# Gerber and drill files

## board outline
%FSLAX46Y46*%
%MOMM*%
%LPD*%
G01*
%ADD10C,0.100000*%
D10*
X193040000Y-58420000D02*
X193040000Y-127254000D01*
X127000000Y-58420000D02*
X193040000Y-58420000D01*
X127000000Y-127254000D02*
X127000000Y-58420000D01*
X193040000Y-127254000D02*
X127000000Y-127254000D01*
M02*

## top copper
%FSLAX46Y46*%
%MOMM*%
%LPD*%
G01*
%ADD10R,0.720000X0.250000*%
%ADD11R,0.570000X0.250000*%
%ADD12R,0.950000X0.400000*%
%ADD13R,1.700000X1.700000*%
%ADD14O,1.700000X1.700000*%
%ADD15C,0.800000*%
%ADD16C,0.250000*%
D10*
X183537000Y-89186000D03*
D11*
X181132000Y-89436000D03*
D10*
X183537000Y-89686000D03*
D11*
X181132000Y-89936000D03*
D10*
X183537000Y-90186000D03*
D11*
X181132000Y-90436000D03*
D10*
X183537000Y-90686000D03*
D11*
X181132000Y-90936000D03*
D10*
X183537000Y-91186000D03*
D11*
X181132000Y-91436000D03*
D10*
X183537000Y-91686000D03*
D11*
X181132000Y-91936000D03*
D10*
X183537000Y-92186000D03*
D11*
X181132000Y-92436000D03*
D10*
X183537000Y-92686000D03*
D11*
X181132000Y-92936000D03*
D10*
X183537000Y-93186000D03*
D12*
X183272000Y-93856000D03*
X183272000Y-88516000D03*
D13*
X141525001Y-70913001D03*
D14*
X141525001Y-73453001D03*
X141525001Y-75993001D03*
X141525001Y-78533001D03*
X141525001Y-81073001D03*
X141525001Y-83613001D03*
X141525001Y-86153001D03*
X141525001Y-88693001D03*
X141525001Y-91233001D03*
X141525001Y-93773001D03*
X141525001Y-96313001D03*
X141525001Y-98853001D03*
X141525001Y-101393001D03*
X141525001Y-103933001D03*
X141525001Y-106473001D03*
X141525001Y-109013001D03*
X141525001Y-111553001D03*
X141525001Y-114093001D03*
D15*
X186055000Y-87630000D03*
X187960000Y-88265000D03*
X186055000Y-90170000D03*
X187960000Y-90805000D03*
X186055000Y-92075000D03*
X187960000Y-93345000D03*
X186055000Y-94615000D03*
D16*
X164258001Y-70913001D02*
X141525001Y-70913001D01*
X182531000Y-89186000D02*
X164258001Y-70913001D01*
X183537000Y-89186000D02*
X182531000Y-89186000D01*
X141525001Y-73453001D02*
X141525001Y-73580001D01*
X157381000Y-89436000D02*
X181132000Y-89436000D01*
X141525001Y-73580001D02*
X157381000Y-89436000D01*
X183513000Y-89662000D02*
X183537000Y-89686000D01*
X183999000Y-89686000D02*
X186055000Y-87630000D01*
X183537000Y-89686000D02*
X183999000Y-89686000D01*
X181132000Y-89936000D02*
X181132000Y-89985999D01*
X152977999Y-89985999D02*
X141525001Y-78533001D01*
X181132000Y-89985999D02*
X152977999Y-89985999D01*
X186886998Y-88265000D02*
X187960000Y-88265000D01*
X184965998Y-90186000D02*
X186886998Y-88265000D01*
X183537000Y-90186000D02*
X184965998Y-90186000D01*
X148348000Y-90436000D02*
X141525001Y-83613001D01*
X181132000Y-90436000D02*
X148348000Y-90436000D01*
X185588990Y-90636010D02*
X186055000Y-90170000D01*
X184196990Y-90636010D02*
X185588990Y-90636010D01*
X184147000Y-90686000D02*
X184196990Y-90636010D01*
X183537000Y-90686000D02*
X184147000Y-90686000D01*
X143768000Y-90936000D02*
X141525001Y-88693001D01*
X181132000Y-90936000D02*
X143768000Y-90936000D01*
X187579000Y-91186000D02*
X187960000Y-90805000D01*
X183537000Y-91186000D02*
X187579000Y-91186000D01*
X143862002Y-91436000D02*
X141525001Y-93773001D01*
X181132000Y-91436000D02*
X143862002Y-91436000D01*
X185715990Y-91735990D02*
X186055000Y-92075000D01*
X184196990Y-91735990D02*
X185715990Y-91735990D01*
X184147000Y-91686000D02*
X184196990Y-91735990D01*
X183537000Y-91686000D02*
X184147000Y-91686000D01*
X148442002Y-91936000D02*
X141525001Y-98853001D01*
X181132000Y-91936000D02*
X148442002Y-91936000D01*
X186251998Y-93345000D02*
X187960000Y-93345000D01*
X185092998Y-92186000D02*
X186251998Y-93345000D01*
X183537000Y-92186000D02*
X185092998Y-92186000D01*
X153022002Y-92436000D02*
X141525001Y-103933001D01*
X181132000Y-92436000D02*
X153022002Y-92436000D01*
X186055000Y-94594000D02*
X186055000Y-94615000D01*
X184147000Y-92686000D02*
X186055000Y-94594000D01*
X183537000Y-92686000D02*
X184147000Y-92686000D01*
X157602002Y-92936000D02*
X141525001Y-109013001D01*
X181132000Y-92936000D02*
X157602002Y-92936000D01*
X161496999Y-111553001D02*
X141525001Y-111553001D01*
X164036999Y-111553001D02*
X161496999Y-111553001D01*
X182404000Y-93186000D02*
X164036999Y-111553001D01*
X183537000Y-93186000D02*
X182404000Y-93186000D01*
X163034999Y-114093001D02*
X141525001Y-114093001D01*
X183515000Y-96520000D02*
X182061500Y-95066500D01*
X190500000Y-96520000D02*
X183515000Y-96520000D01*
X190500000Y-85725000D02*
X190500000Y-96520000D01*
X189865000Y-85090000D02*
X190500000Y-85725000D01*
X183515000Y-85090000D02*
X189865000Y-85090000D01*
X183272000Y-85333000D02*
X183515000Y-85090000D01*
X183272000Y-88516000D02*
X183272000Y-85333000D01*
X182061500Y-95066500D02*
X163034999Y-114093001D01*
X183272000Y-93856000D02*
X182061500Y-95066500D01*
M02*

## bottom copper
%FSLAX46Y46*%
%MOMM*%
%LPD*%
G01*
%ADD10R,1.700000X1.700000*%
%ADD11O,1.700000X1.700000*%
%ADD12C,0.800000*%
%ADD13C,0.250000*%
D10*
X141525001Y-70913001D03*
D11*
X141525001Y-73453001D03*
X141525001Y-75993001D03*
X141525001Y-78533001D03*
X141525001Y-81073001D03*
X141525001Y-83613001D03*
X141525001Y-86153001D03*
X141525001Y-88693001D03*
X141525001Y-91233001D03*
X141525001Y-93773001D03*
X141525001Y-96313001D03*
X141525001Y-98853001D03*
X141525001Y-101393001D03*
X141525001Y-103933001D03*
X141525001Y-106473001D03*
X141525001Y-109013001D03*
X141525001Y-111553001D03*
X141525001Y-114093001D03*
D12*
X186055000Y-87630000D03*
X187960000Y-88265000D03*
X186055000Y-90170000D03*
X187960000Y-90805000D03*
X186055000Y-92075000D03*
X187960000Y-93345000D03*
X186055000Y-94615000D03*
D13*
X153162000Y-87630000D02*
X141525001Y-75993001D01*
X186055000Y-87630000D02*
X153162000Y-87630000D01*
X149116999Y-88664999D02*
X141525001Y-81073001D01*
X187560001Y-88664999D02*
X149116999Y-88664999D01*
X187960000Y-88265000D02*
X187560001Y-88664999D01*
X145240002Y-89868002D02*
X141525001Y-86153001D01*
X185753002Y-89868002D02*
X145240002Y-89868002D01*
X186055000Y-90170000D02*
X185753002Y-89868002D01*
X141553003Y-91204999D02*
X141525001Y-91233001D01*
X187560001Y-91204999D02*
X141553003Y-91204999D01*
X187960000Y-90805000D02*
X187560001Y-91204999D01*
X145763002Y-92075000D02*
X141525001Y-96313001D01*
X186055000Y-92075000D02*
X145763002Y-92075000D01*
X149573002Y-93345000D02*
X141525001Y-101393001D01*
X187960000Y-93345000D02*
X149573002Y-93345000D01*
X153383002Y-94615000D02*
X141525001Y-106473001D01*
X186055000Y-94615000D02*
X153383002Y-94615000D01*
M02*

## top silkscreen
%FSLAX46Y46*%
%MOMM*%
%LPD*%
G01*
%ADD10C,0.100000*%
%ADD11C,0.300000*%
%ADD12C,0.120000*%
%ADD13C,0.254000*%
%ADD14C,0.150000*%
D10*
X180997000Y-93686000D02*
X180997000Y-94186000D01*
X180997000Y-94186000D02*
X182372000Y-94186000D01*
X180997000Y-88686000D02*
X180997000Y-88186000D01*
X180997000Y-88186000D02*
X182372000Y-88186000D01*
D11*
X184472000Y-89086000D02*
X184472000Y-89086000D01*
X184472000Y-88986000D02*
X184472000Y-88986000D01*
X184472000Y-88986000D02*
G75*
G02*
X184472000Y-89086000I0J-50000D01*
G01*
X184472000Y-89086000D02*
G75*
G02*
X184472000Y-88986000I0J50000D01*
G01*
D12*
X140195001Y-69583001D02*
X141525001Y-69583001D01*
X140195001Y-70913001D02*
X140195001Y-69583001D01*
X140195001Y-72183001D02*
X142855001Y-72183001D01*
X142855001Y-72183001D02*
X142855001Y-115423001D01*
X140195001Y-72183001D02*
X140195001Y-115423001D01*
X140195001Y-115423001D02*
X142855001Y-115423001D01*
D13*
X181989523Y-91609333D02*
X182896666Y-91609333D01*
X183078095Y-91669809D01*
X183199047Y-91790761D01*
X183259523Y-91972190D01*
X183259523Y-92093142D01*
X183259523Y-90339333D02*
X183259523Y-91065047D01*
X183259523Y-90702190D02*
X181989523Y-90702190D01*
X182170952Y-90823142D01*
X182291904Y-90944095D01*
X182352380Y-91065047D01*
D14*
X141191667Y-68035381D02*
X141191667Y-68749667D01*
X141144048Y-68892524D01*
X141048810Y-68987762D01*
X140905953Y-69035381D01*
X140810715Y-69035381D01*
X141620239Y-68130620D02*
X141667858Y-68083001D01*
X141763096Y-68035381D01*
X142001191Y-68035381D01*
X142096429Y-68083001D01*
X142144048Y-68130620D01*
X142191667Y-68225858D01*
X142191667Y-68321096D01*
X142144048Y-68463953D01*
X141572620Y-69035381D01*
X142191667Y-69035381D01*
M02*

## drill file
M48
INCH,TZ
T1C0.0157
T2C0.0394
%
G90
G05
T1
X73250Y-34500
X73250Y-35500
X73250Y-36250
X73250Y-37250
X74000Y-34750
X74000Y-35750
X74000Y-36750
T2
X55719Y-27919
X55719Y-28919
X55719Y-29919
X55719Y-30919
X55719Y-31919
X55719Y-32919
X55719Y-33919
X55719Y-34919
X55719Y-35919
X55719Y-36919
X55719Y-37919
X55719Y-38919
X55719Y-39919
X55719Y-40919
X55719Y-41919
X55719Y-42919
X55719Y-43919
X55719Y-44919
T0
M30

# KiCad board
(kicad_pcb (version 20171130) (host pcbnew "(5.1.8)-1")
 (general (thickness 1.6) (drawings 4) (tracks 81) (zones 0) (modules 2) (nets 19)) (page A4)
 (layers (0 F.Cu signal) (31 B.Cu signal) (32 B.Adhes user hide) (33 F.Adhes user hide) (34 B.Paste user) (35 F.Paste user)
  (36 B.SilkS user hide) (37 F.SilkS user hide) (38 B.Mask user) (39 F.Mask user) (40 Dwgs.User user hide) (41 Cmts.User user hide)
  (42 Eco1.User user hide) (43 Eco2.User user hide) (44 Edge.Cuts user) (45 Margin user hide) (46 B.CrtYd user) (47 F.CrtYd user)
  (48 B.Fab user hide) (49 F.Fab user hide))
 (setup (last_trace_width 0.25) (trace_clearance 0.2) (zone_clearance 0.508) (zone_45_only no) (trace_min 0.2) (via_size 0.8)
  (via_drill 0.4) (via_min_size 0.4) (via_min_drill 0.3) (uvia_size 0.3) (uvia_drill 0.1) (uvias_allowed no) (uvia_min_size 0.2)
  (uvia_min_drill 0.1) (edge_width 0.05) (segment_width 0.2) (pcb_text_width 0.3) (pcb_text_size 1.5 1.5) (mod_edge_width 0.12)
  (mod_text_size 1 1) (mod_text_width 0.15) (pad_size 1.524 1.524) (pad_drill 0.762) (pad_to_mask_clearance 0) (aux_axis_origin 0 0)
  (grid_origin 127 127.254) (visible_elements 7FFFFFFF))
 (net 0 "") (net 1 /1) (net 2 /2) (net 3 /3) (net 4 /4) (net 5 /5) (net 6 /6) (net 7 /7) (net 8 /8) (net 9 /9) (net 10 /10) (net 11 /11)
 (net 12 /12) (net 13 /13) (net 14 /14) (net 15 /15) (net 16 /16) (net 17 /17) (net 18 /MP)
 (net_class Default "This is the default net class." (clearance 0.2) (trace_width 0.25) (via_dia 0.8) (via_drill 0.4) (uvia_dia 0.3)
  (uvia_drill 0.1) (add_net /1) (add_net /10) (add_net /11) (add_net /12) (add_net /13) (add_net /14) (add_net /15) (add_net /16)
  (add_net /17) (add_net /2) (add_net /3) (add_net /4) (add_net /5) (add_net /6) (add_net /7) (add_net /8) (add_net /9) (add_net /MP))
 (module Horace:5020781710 (layer F.Cu) (at 182.372 91.186 90)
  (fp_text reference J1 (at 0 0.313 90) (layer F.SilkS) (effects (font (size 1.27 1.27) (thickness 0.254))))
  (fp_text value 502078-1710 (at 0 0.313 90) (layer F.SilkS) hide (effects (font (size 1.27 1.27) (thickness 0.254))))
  (fp_line (start -2.5 -1.375) (end -3 -1.375) (layer F.SilkS) (width 0.1))
  (fp_line (start -3 -1.375) (end -3 0) (layer F.SilkS) (width 0.1))
  (fp_line (start 2.5 -1.375) (end 3 -1.375) (layer F.SilkS) (width 0.1))
  (fp_line (start 3 -1.375) (end 3 0) (layer F.SilkS) (width 0.1))
  (fp_line (start 2.1 2.1) (end 2.1 2.1) (layer F.SilkS) (width 0.3))
  (fp_line (start 2.2 2.1) (end 2.2 2.1) (layer F.SilkS) (width 0.3))
  (fp_arc (start 2.15 2.1) (end 2.1 2.1) (angle -180) (layer F.SilkS) (width 0.3))
  (fp_arc (start 2.15 2.1) (end 2.2 2.1) (angle -180) (layer F.SilkS) (width 0.3))
  (pad 1 smd rect (at 2 1.165 90) (size 0.25 0.72) (layers F.Cu F.Paste F.Mask) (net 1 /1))
  (pad 2 smd rect (at 1.75 -1.24 90) (size 0.25 0.57) (layers F.Cu F.Paste F.Mask) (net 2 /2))
  (pad 3 smd rect (at 1.5 1.165 90) (size 0.25 0.72) (layers F.Cu F.Paste F.Mask) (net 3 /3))
  (pad 4 smd rect (at 1.25 -1.24 90) (size 0.25 0.57) (layers F.Cu F.Paste F.Mask) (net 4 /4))
  (pad 5 smd rect (at 1 1.165 90) (size 0.25 0.72) (layers F.Cu F.Paste F.Mask) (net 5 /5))
  (pad 6 smd rect (at 0.75 -1.24 90) (size 0.25 0.57) (layers F.Cu F.Paste F.Mask) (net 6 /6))
  (pad 7 smd rect (at 0.5 1.165 90) (size 0.25 0.72) (layers F.Cu F.Paste F.Mask) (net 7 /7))
  (pad 8 smd rect (at 0.25 -1.24 90) (size 0.25 0.57) (layers F.Cu F.Paste F.Mask) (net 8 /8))
  (pad 9 smd rect (at 0 1.165 90) (size 0.25 0.72) (layers F.Cu F.Paste F.Mask) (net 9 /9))
  (pad 10 smd rect (at -0.25 -1.24 90) (size 0.25 0.57) (layers F.Cu F.Paste F.Mask) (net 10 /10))
  (pad 11 smd rect (at -0.5 1.165 90) (size 0.25 0.72) (layers F.Cu F.Paste F.Mask) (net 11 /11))
  (pad 12 smd rect (at -0.75 -1.24 90) (size 0.25 0.57) (layers F.Cu F.Paste F.Mask) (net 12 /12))
  (pad 13 smd rect (at -1 1.165 90) (size 0.25 0.72) (layers F.Cu F.Paste F.Mask) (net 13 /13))
  (pad 14 smd rect (at -1.25 -1.24 90) (size 0.25 0.57) (layers F.Cu F.Paste F.Mask) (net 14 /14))
  (pad 15 smd rect (at -1.5 1.165 90) (size 0.25 0.72) (layers F.Cu F.Paste F.Mask) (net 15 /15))
  (pad 16 smd rect (at -1.75 -1.24 90) (size 0.25 0.57) (layers F.Cu F.Paste F.Mask) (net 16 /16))
  (pad 17 smd rect (at -2 1.165 90) (size 0.25 0.72) (layers F.Cu F.Paste F.Mask) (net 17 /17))
  (pad MP1 smd rect (at -2.67 0.9 90) (size 0.4 0.95) (layers F.Cu F.Paste F.Mask) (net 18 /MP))
  (pad MP2 smd rect (at 2.67 0.9 90) (size 0.4 0.95) (layers F.Cu F.Paste F.Mask) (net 18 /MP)))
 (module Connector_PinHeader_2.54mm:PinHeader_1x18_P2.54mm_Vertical (layer F.Cu) (at 141.525001 70.913001)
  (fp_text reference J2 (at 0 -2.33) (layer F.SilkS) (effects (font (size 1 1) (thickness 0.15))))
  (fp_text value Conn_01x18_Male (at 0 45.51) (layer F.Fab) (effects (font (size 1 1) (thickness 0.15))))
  (fp_line (start -1.33 -1.33) (end 0 -1.33) (layer F.SilkS) (width 0.12))
  (fp_line (start -1.33 0) (end -1.33 -1.33) (layer F.SilkS) (width 0.12))
  (fp_line (start -1.33 1.27) (end 1.33 1.27) (layer F.SilkS) (width 0.12))
  (fp_line (start 1.33 1.27) (end 1.33 44.51) (layer F.SilkS) (width 0.12))
  (fp_line (start -1.33 1.27) (end -1.33 44.51) (layer F.SilkS) (width 0.12))
  (fp_line (start -1.33 44.51) (end 1.33 44.51) (layer F.SilkS) (width 0.12))
  (pad 1 thru_hole rect (at 0 0) (size 1.7 1.7) (drill 1) (layers *.Cu *.Mask) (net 1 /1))
  (pad 2 thru_hole oval (at 0 2.54) (size 1.7 1.7) (drill 1) (layers *.Cu *.Mask) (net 2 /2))
  (pad 3 thru_hole oval (at 0 5.08) (size 1.7 1.7) (drill 1) (layers *.Cu *.Mask) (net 3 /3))
  (pad 4 thru_hole oval (at 0 7.62) (size 1.7 1.7) (drill 1) (layers *.Cu *.Mask) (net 4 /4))
  (pad 5 thru_hole oval (at 0 10.16) (size 1.7 1.7) (drill 1) (layers *.Cu *.Mask) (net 5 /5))
  (pad 6 thru_hole oval (at 0 12.7) (size 1.7 1.7) (drill 1) (layers *.Cu *.Mask) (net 6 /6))
  (pad 7 thru_hole oval (at 0 15.24) (size 1.7 1.7) (drill 1) (layers *.Cu *.Mask) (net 7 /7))
  (pad 8 thru_hole oval (at 0 17.78) (size 1.7 1.7) (drill 1) (layers *.Cu *.Mask) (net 8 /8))
  (pad 9 thru_hole oval (at 0 20.32) (size 1.7 1.7) (drill 1) (layers *.Cu *.Mask) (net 9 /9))
  (pad 10 thru_hole oval (at 0 22.86) (size 1.7 1.7) (drill 1) (layers *.Cu *.Mask) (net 10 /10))
  (pad 11 thru_hole oval (at 0 25.4) (size 1.7 1.7) (drill 1) (layers *.Cu *.Mask) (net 11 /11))
  (pad 12 thru_hole oval (at 0 27.94) (size 1.7 1.7) (drill 1) (layers *.Cu *.Mask) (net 12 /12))
  (pad 13 thru_hole oval (at 0 30.48) (size 1.7 1.7) (drill 1) (layers *.Cu *.Mask) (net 13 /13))
  (pad 14 thru_hole oval (at 0 33.02) (size 1.7 1.7) (drill 1) (layers *.Cu *.Mask) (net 14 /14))
  (pad 15 thru_hole oval (at 0 35.56) (size 1.7 1.7) (drill 1) (layers *.Cu *.Mask) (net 15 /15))
  (pad 16 thru_hole oval (at 0 38.1) (size 1.7 1.7) (drill 1) (layers *.Cu *.Mask) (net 16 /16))
  (pad 17 thru_hole oval (at 0 40.64) (size 1.7 1.7) (drill 1) (layers *.Cu *.Mask) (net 17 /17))
  (pad 18 thru_hole oval (at 0 43.18) (size 1.7 1.7) (drill 1) (layers *.Cu *.Mask) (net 18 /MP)))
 (gr_line (start 193.04 58.42) (end 193.04 127.254) (layer Edge.Cuts) (width 0.1))
 (gr_line (start 127 58.42) (end 193.04 58.42) (layer Edge.Cuts) (width 0.1))
 (gr_line (start 127 127.254) (end 127 58.42) (layer Edge.Cuts) (width 0.1))
 (gr_line (start 193.04 127.254) (end 127 127.254) (layer Edge.Cuts) (width 0.1))
 (segment (start 164.258001 70.913001) (end 141.525001 70.913001) (width 0.25) (layer F.Cu) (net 1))
 (segment (start 182.531 89.186) (end 164.258001 70.913001) (width 0.25) (layer F.Cu) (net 1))
 (segment (start 183.537 89.186) (end 182.531 89.186) (width 0.25) (layer F.Cu) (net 1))
 (segment (start 141.525001 73.453001) (end 141.525001 73.580001) (width 0.25) (layer F.Cu) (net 2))
 (segment (start 157.381 89.436) (end 181.132 89.436) (width 0.25) (layer F.Cu) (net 2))
 (segment (start 141.525001 73.580001) (end 157.381 89.436) (width 0.25) (layer F.Cu) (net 2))
 (via (at 186.055 87.63) (size 0.8) (drill 0.4) (layers F.Cu B.Cu) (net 3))
 (segment (start 183.513 89.662) (end 183.537 89.686) (width 0.25) (layer F.Cu) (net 3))
 (segment (start 183.999 89.686) (end 186.055 87.63) (width 0.25) (layer F.Cu) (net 3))
 (segment (start 183.537 89.686) (end 183.999 89.686) (width 0.25) (layer F.Cu) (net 3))
 (segment (start 153.162 87.63) (end 141.525001 75.993001) (width 0.25) (layer B.Cu) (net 3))
 (segment (start 186.055 87.63) (end 153.162 87.63) (width 0.25) (layer B.Cu) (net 3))
 (segment (start 181.132 89.936) (end 181.132 89.985999) (width 0.25) (layer F.Cu) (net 4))
 (segment (start 152.977999 89.985999) (end 141.525001 78.533001) (width 0.25) (layer F.Cu) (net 4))
 (segment (start 181.132 89.985999) (end 152.977999 89.985999) (width 0.25) (layer F.Cu) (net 4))
 (via (at 187.96 88.265) (size 0.8) (drill 0.4) (layers F.Cu B.Cu) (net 5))
 (segment (start 186.886998 88.265) (end 187.96 88.265) (width 0.25) (layer F.Cu) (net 5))
 (segment (start 184.965998 90.186) (end 186.886998 88.265) (width 0.25) (layer F.Cu) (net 5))
 (segment (start 183.537 90.186) (end 184.965998 90.186) (width 0.25) (layer F.Cu) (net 5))
 (segment (start 149.116999 88.664999) (end 141.525001 81.073001) (width 0.25) (layer B.Cu) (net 5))
 (segment (start 187.560001 88.664999) (end 149.116999 88.664999) (width 0.25) (layer B.Cu) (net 5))
 (segment (start 187.96 88.265) (end 187.560001 88.664999) (width 0.25) (layer B.Cu) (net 5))
 (segment (start 148.348 90.436) (end 141.525001 83.613001) (width 0.25) (layer F.Cu) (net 6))
 (segment (start 181.132 90.436) (end 148.348 90.436) (width 0.25) (layer F.Cu) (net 6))
 (via (at 186.055 90.17) (size 0.8) (drill 0.4) (layers F.Cu B.Cu) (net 7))
 (segment (start 185.58899 90.63601) (end 186.055 90.17) (width 0.25) (layer F.Cu) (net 7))
 (segment (start 184.19699 90.63601) (end 185.58899 90.63601) (width 0.25) (layer F.Cu) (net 7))
 (segment (start 184.147 90.686) (end 184.19699 90.63601) (width 0.25) (layer F.Cu) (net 7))
 (segment (start 183.537 90.686) (end 184.147 90.686) (width 0.25) (layer F.Cu) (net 7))
 (segment (start 145.240002 89.868002) (end 141.525001 86.153001) (width 0.25) (layer B.Cu) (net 7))
 (segment (start 185.753002 89.868002) (end 145.240002 89.868002) (width 0.25) (layer B.Cu) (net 7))
 (segment (start 186.055 90.17) (end 185.753002 89.868002) (width 0.25) (layer B.Cu) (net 7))
 (segment (start 143.768 90.936) (end 141.525001 88.693001) (width 0.25) (layer F.Cu) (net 8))
 (segment (start 181.132 90.936) (end 143.768 90.936) (width 0.25) (layer F.Cu) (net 8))
 (via (at 187.96 90.805) (size 0.8) (drill 0.4) (layers F.Cu B.Cu) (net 9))
 (segment (start 187.579 91.186) (end 187.96 90.805) (width 0.25) (layer F.Cu) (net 9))
 (segment (start 183.537 91.186) (end 187.579 91.186) (width 0.25) (layer F.Cu) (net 9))
 (segment (start 141.553003 91.204999) (end 141.525001 91.233001) (width 0.25) (layer B.Cu) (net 9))
 (segment (start 187.560001 91.204999) (end 141.553003 91.204999) (width 0.25) (layer B.Cu) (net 9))
 (segment (start 187.96 90.805) (end 187.560001 91.204999) (width 0.25) (layer B.Cu) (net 9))
 (segment (start 143.862002 91.436) (end 141.525001 93.773001) (width 0.25) (layer F.Cu) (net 10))
 (segment (start 181.132 91.436) (end 143.862002 91.436) (width 0.25) (layer F.Cu) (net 10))
 (via (at 186.055 92.075) (size 0.8) (drill 0.4) (layers F.Cu B.Cu) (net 11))
 (segment (start 185.71599 91.73599) (end 186.055 92.075) (width 0.25) (layer F.Cu) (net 11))
 (segment (start 184.19699 91.73599) (end 185.71599 91.73599) (width 0.25) (layer F.Cu) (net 11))
 (segment (start 184.147 91.686) (end 184.19699 91.73599) (width 0.25) (layer F.Cu) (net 11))
 (segment (start 183.537 91.686) (end 184.147 91.686) (width 0.25) (layer F.Cu) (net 11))
 (segment (start 145.763002 92.075) (end 141.525001 96.313001) (width 0.25) (layer B.Cu) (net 11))
 (segment (start 186.055 92.075) (end 145.763002 92.075) (width 0.25) (layer B.Cu) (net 11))
 (segment (start 148.442002 91.936) (end 141.525001 98.853001) (width 0.25) (layer F.Cu) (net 12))
 (segment (start 181.132 91.936) (end 148.442002 91.936) (width 0.25) (layer F.Cu) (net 12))
 (via (at 187.96 93.345) (size 0.8) (drill 0.4) (layers F.Cu B.Cu) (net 13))
 (segment (start 186.251998 93.345) (end 187.96 93.345) (width 0.25) (layer F.Cu) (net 13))
 (segment (start 185.092998 92.186) (end 186.251998 93.345) (width 0.25) (layer F.Cu) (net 13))
 (segment (start 183.537 92.186) (end 185.092998 92.186) (width 0.25) (layer F.Cu) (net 13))
 (segment (start 149.573002 93.345) (end 141.525001 101.393001) (width 0.25) (layer B.Cu) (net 13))
 (segment (start 187.96 93.345) (end 149.573002 93.345) (width 0.25) (layer B.Cu) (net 13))
 (segment (start 153.022002 92.436) (end 141.525001 103.933001) (width 0.25) (layer F.Cu) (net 14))
 (segment (start 181.132 92.436) (end 153.022002 92.436) (width 0.25) (layer F.Cu) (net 14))
 (via (at 186.055 94.615) (size 0.8) (drill 0.4) (layers F.Cu B.Cu) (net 15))
 (segment (start 186.055 94.594) (end 186.055 94.615) (width 0.25) (layer F.Cu) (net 15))
 (segment (start 184.147 92.686) (end 186.055 94.594) (width 0.25) (layer F.Cu) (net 15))
 (segment (start 183.537 92.686) (end 184.147 92.686) (width 0.25) (layer F.Cu) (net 15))
 (segment (start 153.383002 94.615) (end 141.525001 106.473001) (width 0.25) (layer B.Cu) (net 15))
 (segment (start 186.055 94.615) (end 153.383002 94.615) (width 0.25) (layer B.Cu) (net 15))
 (segment (start 157.602002 92.936) (end 141.525001 109.013001) (width 0.25) (layer F.Cu) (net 16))
 (segment (start 181.132 92.936) (end 157.602002 92.936) (width 0.25) (layer F.Cu) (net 16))
 (segment (start 161.496999 111.553001) (end 141.525001 111.553001) (width 0.25) (layer F.Cu) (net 17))
 (segment (start 164.036999 111.553001) (end 161.496999 111.553001) (width 0.25) (layer F.Cu) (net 17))
 (segment (start 182.404 93.186) (end 164.036999 111.553001) (width 0.25) (layer F.Cu) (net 17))
 (segment (start 183.537 93.186) (end 182.404 93.186) (width 0.25) (layer F.Cu) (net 17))
 (segment (start 163.034999 114.093001) (end 141.525001 114.093001) (width 0.25) (layer F.Cu) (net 18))
 (segment (start 183.515 96.52) (end 182.0615 95.0665) (width 0.25) (layer F.Cu) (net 18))
 (segment (start 190.5 96.52) (end 183.515 96.52) (width 0.25) (layer F.Cu) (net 18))
 (segment (start 190.5 85.725) (end 190.5 96.52) (width 0.25) (layer F.Cu) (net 18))
 (segment (start 189.865 85.09) (end 190.5 85.725) (width 0.25) (layer F.Cu) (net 18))
 (segment (start 183.515 85.09) (end 189.865 85.09) (width 0.25) (layer F.Cu) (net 18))
 (segment (start 183.272 85.333) (end 183.515 85.09) (width 0.25) (layer F.Cu) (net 18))
 (segment (start 183.272 88.516) (end 183.272 85.333) (width 0.25) (layer F.Cu) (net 18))
 (segment (start 182.0615 95.0665) (end 163.034999 114.093001) (width 0.25) (layer F.Cu) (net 18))
 (segment (start 183.272 93.856) (end 182.0615 95.0665) (width 0.25) (layer F.Cu) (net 18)))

